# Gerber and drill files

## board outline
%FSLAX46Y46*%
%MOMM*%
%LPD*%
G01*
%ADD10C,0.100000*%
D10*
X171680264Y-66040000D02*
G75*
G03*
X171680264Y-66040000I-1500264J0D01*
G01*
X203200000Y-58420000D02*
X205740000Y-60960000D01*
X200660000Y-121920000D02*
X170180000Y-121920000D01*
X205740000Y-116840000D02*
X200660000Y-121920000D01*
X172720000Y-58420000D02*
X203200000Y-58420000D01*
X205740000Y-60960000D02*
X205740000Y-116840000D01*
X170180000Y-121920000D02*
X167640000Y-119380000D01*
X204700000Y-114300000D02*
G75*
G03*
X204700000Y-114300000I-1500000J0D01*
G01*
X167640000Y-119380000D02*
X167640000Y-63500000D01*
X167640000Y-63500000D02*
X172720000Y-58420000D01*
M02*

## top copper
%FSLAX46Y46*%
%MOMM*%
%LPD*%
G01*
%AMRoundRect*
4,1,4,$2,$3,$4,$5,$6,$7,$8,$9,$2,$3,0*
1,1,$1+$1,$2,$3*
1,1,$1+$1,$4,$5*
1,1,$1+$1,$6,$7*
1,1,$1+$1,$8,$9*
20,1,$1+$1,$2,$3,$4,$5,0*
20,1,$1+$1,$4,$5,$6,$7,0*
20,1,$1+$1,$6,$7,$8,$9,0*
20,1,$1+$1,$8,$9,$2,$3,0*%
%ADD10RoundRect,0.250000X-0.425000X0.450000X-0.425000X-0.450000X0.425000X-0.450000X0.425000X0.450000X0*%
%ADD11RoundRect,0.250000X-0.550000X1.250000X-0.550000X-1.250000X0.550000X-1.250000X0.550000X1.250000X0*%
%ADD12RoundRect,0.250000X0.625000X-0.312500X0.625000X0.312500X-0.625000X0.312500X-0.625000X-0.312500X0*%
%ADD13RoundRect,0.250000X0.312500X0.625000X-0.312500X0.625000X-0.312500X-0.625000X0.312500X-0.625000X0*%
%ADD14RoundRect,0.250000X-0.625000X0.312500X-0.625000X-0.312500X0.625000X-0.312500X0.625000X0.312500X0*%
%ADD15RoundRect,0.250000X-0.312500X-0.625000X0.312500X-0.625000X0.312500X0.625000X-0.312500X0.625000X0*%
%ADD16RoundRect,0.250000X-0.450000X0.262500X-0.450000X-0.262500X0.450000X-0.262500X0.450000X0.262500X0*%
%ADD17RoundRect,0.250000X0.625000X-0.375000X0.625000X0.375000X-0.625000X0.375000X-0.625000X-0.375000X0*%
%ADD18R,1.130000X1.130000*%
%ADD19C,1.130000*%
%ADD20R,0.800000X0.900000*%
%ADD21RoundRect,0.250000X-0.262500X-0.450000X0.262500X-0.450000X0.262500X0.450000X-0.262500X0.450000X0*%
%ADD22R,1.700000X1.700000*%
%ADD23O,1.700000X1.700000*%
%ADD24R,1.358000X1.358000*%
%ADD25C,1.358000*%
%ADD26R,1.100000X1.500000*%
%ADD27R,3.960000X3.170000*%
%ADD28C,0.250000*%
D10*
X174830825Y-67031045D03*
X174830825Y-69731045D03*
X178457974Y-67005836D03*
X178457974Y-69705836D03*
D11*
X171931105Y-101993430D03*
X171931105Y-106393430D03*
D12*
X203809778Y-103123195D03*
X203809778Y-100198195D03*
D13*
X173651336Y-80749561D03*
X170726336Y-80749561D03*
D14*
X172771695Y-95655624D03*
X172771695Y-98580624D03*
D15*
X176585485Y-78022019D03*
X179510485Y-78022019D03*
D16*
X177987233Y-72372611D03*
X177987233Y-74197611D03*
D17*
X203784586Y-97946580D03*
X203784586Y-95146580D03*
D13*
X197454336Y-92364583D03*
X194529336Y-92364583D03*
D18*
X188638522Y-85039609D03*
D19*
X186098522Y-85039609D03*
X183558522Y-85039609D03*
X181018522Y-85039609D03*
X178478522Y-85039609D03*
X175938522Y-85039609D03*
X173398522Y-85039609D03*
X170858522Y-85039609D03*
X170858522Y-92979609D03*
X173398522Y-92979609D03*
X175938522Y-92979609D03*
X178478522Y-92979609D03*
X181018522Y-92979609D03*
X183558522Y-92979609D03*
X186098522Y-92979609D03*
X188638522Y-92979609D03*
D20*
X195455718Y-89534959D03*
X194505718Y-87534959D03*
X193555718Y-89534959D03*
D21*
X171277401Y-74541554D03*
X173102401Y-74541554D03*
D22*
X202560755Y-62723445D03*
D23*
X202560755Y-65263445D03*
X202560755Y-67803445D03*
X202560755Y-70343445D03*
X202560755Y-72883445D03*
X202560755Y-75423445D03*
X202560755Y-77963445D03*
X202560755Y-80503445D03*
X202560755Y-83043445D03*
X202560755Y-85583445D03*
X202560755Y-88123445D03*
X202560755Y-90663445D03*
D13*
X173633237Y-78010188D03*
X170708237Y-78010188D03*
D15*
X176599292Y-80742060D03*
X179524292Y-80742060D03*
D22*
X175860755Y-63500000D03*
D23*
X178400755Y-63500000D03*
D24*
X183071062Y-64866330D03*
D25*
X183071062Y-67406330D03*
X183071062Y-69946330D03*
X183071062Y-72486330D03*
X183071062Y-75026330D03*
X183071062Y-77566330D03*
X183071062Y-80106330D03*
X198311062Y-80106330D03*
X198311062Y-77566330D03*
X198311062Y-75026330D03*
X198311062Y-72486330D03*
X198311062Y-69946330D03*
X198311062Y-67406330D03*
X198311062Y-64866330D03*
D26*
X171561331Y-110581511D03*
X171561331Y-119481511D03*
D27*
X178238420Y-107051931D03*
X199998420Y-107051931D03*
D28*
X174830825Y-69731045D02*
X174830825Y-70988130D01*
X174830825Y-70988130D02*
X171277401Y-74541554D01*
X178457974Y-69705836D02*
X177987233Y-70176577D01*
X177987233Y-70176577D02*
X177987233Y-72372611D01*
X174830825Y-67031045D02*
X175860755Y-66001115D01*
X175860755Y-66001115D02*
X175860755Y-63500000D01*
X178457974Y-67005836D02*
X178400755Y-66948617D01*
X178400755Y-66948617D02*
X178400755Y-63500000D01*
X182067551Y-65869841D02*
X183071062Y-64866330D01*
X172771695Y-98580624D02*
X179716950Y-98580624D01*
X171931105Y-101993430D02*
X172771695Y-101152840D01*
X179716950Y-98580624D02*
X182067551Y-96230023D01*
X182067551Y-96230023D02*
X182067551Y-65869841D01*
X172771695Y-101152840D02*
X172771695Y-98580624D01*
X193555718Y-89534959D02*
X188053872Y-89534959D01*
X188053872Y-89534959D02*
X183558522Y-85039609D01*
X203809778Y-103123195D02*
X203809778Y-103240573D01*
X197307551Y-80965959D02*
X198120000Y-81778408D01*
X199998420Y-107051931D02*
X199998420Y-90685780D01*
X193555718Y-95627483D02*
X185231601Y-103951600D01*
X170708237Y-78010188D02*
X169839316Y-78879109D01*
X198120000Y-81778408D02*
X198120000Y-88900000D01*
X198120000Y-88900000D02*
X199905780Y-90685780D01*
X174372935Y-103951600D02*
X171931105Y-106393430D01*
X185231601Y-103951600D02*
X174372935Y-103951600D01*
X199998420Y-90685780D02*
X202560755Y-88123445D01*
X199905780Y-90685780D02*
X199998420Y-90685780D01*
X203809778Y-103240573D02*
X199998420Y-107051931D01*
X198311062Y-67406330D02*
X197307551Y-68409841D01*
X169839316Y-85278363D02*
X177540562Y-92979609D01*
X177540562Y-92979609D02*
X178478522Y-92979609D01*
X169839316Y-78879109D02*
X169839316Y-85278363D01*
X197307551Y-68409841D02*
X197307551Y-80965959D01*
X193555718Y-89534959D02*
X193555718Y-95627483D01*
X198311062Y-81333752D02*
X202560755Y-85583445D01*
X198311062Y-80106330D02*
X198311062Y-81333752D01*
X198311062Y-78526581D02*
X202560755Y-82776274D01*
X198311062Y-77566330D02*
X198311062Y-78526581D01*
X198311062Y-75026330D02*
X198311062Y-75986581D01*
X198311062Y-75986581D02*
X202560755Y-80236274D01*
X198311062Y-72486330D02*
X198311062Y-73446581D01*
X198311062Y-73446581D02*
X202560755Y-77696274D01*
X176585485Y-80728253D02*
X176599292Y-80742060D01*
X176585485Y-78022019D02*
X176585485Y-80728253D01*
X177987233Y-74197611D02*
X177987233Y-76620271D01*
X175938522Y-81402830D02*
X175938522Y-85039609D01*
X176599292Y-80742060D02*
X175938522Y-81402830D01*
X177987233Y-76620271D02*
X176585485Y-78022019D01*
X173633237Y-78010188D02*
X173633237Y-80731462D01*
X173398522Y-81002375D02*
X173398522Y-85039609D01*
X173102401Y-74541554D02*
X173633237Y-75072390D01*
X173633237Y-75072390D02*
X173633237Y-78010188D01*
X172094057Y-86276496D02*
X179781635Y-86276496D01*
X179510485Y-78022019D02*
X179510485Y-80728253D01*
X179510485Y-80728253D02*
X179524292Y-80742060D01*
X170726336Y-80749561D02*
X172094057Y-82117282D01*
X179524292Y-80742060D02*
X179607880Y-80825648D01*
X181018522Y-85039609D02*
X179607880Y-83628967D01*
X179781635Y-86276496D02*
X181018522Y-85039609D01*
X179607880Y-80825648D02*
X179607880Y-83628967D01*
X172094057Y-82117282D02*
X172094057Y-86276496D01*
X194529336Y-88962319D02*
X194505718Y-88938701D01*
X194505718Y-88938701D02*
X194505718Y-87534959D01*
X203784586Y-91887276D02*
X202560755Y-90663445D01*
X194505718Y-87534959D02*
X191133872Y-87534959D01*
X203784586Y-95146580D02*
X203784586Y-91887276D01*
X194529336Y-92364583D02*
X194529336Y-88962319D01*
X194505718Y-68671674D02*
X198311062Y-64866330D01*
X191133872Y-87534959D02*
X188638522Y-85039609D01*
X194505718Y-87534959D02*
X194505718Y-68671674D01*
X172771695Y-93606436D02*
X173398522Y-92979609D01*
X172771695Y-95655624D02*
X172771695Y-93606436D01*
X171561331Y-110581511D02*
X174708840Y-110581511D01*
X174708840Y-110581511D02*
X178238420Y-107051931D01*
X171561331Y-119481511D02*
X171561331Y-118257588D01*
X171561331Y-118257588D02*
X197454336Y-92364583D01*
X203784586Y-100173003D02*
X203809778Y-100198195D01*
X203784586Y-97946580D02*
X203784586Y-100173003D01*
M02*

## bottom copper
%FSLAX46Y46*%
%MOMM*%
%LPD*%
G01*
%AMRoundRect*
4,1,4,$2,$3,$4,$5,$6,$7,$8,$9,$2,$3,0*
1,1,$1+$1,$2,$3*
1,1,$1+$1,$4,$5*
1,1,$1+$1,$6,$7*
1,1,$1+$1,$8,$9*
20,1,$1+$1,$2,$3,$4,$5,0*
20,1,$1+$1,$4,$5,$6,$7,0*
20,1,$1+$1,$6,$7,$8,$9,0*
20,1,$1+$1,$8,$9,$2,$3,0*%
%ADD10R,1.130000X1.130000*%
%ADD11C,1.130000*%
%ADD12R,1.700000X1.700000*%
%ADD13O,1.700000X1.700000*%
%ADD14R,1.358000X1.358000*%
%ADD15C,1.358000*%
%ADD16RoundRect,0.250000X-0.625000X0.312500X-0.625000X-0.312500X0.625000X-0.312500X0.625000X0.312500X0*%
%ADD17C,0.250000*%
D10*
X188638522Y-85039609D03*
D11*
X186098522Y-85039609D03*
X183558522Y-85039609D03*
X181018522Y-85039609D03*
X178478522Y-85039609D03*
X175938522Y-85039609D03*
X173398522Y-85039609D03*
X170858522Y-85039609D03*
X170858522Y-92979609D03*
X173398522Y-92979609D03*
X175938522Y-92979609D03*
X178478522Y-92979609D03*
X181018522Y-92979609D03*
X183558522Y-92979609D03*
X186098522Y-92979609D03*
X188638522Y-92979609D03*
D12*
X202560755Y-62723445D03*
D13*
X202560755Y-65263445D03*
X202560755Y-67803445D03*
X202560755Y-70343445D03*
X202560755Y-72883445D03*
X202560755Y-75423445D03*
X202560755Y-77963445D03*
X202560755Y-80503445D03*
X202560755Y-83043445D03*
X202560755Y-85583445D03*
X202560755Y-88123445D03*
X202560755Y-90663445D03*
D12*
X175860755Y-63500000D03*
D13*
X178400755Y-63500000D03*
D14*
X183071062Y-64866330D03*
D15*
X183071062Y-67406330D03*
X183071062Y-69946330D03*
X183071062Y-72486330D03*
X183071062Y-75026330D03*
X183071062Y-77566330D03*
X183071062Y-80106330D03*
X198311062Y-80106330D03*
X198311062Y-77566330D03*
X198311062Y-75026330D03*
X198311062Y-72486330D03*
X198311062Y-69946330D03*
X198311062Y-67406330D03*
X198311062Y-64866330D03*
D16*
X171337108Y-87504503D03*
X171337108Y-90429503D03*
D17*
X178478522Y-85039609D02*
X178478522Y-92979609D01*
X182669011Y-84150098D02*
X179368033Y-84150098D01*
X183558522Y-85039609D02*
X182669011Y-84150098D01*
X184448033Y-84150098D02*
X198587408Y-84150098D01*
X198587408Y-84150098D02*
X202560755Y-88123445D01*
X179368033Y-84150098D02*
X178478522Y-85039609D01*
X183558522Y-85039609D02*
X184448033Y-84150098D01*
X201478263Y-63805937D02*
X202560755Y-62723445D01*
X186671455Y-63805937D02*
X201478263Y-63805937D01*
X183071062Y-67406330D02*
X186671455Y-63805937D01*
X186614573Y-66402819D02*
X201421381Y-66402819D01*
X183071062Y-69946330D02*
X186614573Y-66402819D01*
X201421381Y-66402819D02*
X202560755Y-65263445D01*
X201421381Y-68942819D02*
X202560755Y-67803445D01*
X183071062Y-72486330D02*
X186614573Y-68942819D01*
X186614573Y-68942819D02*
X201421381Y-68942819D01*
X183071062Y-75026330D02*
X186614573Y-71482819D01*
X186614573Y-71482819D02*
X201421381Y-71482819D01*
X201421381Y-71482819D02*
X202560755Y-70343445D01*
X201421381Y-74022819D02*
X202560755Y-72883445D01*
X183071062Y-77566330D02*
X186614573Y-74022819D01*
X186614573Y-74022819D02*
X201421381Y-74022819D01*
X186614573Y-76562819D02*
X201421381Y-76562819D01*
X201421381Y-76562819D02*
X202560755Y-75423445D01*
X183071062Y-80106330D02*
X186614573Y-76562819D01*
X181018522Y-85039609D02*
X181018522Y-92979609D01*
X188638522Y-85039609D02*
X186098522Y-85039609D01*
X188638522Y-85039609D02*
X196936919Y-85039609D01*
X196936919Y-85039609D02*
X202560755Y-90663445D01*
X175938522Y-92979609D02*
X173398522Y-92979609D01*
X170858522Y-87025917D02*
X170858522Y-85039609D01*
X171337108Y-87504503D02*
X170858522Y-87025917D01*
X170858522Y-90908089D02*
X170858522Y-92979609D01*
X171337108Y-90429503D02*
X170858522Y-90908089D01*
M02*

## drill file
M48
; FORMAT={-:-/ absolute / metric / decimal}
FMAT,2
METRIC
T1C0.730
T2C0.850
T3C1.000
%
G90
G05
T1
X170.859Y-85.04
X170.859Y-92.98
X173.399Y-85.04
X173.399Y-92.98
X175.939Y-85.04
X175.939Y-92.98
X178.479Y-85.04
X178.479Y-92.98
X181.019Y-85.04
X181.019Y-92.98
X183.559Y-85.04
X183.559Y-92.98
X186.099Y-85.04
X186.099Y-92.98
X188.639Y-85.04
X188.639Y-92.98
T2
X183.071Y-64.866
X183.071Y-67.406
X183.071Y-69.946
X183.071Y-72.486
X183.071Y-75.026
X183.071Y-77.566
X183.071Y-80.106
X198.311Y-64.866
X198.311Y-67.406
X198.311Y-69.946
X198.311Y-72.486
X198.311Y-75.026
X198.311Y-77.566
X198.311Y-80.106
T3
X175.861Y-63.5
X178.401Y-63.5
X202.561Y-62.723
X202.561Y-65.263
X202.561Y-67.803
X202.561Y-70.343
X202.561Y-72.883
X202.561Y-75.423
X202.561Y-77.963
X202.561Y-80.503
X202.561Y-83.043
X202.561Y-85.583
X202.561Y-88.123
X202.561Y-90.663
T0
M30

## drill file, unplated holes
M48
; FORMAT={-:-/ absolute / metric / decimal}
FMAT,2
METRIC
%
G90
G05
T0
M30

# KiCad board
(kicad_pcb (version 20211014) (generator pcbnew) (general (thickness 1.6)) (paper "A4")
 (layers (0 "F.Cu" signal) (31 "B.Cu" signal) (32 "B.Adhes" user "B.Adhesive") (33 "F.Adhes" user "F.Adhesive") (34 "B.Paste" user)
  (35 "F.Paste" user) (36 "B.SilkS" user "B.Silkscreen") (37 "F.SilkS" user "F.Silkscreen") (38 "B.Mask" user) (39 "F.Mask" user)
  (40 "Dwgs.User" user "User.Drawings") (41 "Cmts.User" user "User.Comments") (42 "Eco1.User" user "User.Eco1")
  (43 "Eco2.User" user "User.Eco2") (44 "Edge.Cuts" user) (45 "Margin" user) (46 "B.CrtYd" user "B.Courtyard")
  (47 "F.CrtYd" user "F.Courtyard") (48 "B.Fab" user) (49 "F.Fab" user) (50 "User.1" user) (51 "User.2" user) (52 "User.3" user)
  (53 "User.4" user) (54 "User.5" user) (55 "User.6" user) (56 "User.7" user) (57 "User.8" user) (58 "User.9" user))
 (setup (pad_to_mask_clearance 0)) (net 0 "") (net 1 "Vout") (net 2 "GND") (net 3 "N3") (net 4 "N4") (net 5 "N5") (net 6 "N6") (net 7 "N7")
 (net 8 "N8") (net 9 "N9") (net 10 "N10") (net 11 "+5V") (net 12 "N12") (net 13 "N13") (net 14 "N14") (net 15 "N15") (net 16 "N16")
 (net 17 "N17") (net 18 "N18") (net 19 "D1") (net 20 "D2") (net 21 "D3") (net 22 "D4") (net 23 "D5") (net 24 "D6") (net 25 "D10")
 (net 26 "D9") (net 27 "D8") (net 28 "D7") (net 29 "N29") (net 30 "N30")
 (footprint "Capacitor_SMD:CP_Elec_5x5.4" (layer "F.Cu") (at 171.931105 104.19343 -90)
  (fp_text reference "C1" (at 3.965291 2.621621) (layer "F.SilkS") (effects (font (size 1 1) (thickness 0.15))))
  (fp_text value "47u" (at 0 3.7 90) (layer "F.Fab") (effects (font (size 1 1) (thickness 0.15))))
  (pad "1" smd roundrect (at -2.2 0 270) (size 3 1.6) (layers "F.Cu" "F.Paste" "F.Mask") (roundrect_rratio 0.15625) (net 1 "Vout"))
  (pad "2" smd roundrect (at 2.2 0 270) (size 3 1.6) (layers "F.Cu" "F.Paste" "F.Mask") (roundrect_rratio 0.15625) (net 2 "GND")))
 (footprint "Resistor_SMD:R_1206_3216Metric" (layer "F.Cu") (at 203.809778 101.660695 90)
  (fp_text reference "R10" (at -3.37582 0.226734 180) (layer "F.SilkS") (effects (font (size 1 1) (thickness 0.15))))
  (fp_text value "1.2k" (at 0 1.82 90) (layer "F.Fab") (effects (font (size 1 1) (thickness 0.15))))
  (pad "1" smd roundrect (at -1.4625 0 90) (size 1.125 1.75) (layers "F.Cu" "F.Paste" "F.Mask") (roundrect_rratio 0.2222222222)
   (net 2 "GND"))
  (pad "2" smd roundrect (at 1.4625 0 90) (size 1.125 1.75) (layers "F.Cu" "F.Paste" "F.Mask") (roundrect_rratio 0.2222222222) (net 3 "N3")))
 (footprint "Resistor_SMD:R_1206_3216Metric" (layer "F.Cu") (at 172.188836 80.749561 180)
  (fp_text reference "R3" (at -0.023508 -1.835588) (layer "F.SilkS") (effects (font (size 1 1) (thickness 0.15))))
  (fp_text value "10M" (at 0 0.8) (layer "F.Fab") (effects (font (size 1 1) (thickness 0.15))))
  (pad "1" smd roundrect (at -1.4625 0 180) (size 1.125 1.75) (layers "F.Cu" "F.Paste" "F.Mask") (roundrect_rratio 0.2222222222)
   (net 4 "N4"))
  (pad "2" smd roundrect (at 1.4625 0 180) (size 1.125 1.75) (layers "F.Cu" "F.Paste" "F.Mask") (roundrect_rratio 0.2222222222) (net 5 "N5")))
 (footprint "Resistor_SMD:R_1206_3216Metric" (layer "F.Cu") (at 172.771695 97.118124 -90)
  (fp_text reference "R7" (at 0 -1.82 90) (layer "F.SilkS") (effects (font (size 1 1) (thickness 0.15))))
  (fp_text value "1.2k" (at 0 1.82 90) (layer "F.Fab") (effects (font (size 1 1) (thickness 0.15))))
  (pad "1" smd roundrect (at -1.4625 0 270) (size 1.125 1.75) (layers "F.Cu" "F.Paste" "F.Mask") (roundrect_rratio 0.2222222222)
   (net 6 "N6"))
  (pad "2" smd roundrect (at 1.4625 0 270) (size 1.125 1.75) (layers "F.Cu" "F.Paste" "F.Mask") (roundrect_rratio 0.2222222222)
   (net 1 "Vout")))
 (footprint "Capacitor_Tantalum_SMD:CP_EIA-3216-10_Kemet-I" (layer "F.Cu") (at 174.830825 68.381045 -90)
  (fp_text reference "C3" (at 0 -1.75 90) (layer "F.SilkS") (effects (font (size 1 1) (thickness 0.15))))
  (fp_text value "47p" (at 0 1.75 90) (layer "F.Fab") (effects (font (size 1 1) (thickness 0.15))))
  (pad "1" smd roundrect (at -1.35 0 270) (size 1.4 1.35) (layers "F.Cu" "F.Paste" "F.Mask") (roundrect_rratio 0.1851851852) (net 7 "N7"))
  (pad "2" smd roundrect (at 1.35 0 270) (size 1.4 1.35) (layers "F.Cu" "F.Paste" "F.Mask") (roundrect_rratio 0.1851851852) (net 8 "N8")))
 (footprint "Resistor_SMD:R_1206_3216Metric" (layer "F.Cu") (at 178.047985 78.022019)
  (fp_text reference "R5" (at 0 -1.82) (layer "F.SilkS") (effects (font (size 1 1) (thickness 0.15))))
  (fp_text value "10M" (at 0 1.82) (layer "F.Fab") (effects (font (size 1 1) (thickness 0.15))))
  (pad "1" smd roundrect (at -1.4625 0) (size 1.125 1.75) (layers "F.Cu" "F.Paste" "F.Mask") (roundrect_rratio 0.2222222222) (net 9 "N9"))
  (pad "2" smd roundrect (at 1.4625 0) (size 1.125 1.75) (layers "F.Cu" "F.Paste" "F.Mask") (roundrect_rratio 0.2222222222) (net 5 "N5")))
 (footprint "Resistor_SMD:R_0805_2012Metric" (layer "F.Cu") (at 177.987233 73.285111 -90)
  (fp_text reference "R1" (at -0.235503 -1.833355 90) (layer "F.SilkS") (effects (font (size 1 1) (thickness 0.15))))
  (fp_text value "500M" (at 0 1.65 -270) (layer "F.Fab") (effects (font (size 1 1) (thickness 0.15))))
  (pad "1" smd roundrect (at -0.9125 0 270) (size 1.025 1.4) (layers "F.Cu" "F.Paste" "F.Mask") (roundrect_rratio 0.243902439)
   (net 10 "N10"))
  (pad "2" smd roundrect (at 0.9125 0 270) (size 1.025 1.4) (layers "F.Cu" "F.Paste" "F.Mask") (roundrect_rratio 0.243902439) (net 9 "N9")))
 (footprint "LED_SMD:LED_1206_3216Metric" (layer "F.Cu") (at 203.784586 96.54658 90)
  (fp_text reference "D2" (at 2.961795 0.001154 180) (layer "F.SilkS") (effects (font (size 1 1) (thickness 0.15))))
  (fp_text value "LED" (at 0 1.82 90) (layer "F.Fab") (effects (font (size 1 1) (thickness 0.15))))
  (pad "1" smd roundrect (at -1.4 0 90) (size 1.25 1.75) (layers "F.Cu" "F.Paste" "F.Mask") (roundrect_rratio 0.2) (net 3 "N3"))
  (pad "2" smd roundrect (at 1.4 0 90) (size 1.25 1.75) (layers "F.Cu" "F.Paste" "F.Mask") (roundrect_rratio 0.2) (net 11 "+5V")))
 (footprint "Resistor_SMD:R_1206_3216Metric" (layer "F.Cu") (at 195.991836 92.364583 180)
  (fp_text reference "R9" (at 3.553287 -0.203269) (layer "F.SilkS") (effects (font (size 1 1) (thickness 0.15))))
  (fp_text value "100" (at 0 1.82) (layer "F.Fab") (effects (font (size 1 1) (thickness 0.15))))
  (pad "1" smd roundrect (at -1.4625 0 180) (size 1.125 1.75) (layers "F.Cu" "F.Paste" "F.Mask") (roundrect_rratio 0.2222222222)
   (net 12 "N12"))
  (pad "2" smd roundrect (at 1.4625 0 180) (size 1.125 1.75) (layers "F.Cu" "F.Paste" "F.Mask") (roundrect_rratio 0.2222222222)
   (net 11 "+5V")))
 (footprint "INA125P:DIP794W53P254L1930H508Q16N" (layer "F.Cu") (at 179.748522 89.009609 -90)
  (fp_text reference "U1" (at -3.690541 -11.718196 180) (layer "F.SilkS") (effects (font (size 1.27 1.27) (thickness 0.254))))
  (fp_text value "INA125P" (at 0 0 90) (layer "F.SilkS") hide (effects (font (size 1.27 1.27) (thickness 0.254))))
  (pad "1" thru_hole rect locked (at -3.97 -8.89 270) (size 1.13 1.13) (drill 0.73) (layers *.Cu *.Mask) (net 11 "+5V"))
  (pad "2" thru_hole circle locked (at -3.97 -6.35 270) (size 1.13 1.13) (drill 0.73) (layers *.Cu *.Mask) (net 11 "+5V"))
  (pad "3" thru_hole circle locked (at -3.97 -3.81 270) (size 1.13 1.13) (drill 0.73) (layers *.Cu *.Mask) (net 2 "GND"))
  (pad "4" thru_hole circle locked (at -3.97 -1.27 270) (size 1.13 1.13) (drill 0.73) (layers *.Cu *.Mask) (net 5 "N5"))
  (pad "5" thru_hole circle locked (at -3.97 1.27 270) (size 1.13 1.13) (drill 0.73) (layers *.Cu *.Mask) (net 2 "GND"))
  (pad "6" thru_hole circle locked (at -3.97 3.81 270) (size 1.13 1.13) (drill 0.73) (layers *.Cu *.Mask) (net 9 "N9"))
  (pad "7" thru_hole circle locked (at -3.97 6.35 270) (size 1.13 1.13) (drill 0.73) (layers *.Cu *.Mask) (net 4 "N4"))
  (pad "8" thru_hole circle locked (at -3.97 8.89 270) (size 1.13 1.13) (drill 0.73) (layers *.Cu *.Mask) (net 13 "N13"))
  (pad "9" thru_hole circle locked (at 3.97 8.89 270) (size 1.13 1.13) (drill 0.73) (layers *.Cu *.Mask) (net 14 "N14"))
  (pad "10" thru_hole circle locked (at 3.97 6.35 270) (size 1.13 1.13) (drill 0.73) (layers *.Cu *.Mask) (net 6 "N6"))
  (pad "11" thru_hole circle locked (at 3.97 3.81 270) (size 1.13 1.13) (drill 0.73) (layers *.Cu *.Mask) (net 6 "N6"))
  (pad "12" thru_hole circle locked (at 3.97 1.27 270) (size 1.13 1.13) (drill 0.73) (layers *.Cu *.Mask) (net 2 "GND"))
  (pad "13" thru_hole circle locked (at 3.97 -1.27 270) (size 1.13 1.13) (drill 0.73) (layers *.Cu *.Mask) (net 5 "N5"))
  (pad "14" thru_hole circle locked (at 3.97 -3.81 270) (size 1.13 1.13) (drill 0.73) (layers *.Cu *.Mask) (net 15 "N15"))
  (pad "15" thru_hole circle locked (at 3.97 -6.35 270) (size 1.13 1.13) (drill 0.73) (layers *.Cu *.Mask) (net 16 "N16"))
  (pad "16" thru_hole circle locked (at 3.97 -8.89 270) (size 1.13 1.13) (drill 0.73) (layers *.Cu *.Mask) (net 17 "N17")))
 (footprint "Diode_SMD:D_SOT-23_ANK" (layer "F.Cu") (at 194.505718 88.534959 90)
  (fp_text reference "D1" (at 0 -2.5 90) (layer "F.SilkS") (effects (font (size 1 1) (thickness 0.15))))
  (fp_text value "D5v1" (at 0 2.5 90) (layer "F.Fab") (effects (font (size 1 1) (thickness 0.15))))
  (pad "" smd rect (at -1 0.95 90) (size 0.9 0.8) (layers "F.Cu" "F.Paste" "F.Mask"))
  (pad "1" smd rect (at 1 0 90) (size 0.9 0.8) (layers "F.Cu" "F.Paste" "F.Mask") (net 11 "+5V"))
  (pad "2" smd rect (at -1 -0.95 90) (size 0.9 0.8) (layers "F.Cu" "F.Paste" "F.Mask") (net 2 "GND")))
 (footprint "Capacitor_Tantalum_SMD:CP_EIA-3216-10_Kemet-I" (layer "F.Cu") (at 178.457974 68.355836 -90)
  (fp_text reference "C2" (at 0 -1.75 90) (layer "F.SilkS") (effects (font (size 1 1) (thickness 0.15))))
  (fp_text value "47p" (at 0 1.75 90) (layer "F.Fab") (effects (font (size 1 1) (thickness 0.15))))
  (pad "1" smd roundrect (at -1.35 0 270) (size 1.4 1.35) (layers "F.Cu" "F.Paste" "F.Mask") (roundrect_rratio 0.1851851852) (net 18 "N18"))
  (pad "2" smd roundrect (at 1.35 0 270) (size 1.4 1.35) (layers "F.Cu" "F.Paste" "F.Mask") (roundrect_rratio 0.1851851852) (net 10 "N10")))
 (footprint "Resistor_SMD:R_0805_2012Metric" (layer "F.Cu") (at 172.189901 74.541554)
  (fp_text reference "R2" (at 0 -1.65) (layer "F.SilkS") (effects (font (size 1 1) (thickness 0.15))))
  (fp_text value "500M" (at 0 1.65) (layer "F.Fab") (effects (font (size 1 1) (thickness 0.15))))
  (pad "1" smd roundrect (at -0.9125 0) (size 1.025 1.4) (layers "F.Cu" "F.Paste" "F.Mask") (roundrect_rratio 0.243902439) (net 8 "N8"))
  (pad "2" smd roundrect (at 0.9125 0) (size 1.025 1.4) (layers "F.Cu" "F.Paste" "F.Mask") (roundrect_rratio 0.243902439) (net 4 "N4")))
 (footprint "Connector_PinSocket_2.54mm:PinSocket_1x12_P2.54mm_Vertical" (layer "F.Cu") (at 202.560755 62.723445)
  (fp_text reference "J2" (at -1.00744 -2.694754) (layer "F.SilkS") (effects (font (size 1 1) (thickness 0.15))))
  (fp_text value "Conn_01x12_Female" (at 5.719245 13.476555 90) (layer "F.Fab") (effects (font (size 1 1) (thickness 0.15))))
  (pad "1" thru_hole rect (at 0 0) (size 1.7 1.7) (drill 1) (layers *.Cu *.Mask) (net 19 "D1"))
  (pad "2" thru_hole oval (at 0 2.54) (size 1.7 1.7) (drill 1) (layers *.Cu *.Mask) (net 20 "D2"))
  (pad "3" thru_hole oval (at 0 5.08) (size 1.7 1.7) (drill 1) (layers *.Cu *.Mask) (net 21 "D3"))
  (pad "4" thru_hole oval (at 0 7.62) (size 1.7 1.7) (drill 1) (layers *.Cu *.Mask) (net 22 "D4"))
  (pad "5" thru_hole oval (at 0 10.16) (size 1.7 1.7) (drill 1) (layers *.Cu *.Mask) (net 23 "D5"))
  (pad "6" thru_hole oval (at 0 12.7) (size 1.7 1.7) (drill 1) (layers *.Cu *.Mask) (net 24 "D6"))
  (pad "7" thru_hole oval (at 0 15.24) (size 1.7 1.7) (drill 1) (layers *.Cu *.Mask) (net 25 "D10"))
  (pad "8" thru_hole oval (at 0 17.78) (size 1.7 1.7) (drill 1) (layers *.Cu *.Mask) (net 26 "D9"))
  (pad "9" thru_hole oval (at 0 20.32) (size 1.7 1.7) (drill 1) (layers *.Cu *.Mask) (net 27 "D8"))
  (pad "10" thru_hole oval (at 0 22.86) (size 1.7 1.7) (drill 1) (layers *.Cu *.Mask) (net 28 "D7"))
  (pad "11" thru_hole oval (at 0 25.4) (size 1.7 1.7) (drill 1) (layers *.Cu *.Mask) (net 2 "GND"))
  (pad "12" thru_hole oval (at 0 27.94) (size 1.7 1.7) (drill 1) (layers *.Cu *.Mask) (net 11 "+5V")))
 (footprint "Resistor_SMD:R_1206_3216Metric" (layer "F.Cu") (at 172.170737 78.010188 180)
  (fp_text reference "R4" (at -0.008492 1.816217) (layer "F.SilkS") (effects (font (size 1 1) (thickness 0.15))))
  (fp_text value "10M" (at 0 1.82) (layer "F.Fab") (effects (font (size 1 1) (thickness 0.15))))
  (pad "1" smd roundrect (at -1.4625 0 180) (size 1.125 1.75) (layers "F.Cu" "F.Paste" "F.Mask") (roundrect_rratio 0.2222222222)
   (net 4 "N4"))
  (pad "2" smd roundrect (at 1.4625 0 180) (size 1.125 1.75) (layers "F.Cu" "F.Paste" "F.Mask") (roundrect_rratio 0.2222222222)
   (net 2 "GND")))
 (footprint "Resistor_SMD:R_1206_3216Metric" (layer "F.Cu") (at 178.061792 80.74206)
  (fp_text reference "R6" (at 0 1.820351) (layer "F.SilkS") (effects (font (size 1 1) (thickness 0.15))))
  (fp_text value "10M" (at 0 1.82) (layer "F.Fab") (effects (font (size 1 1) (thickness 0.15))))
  (pad "1" smd roundrect (at -1.4625 0) (size 1.125 1.75) (layers "F.Cu" "F.Paste" "F.Mask") (roundrect_rratio 0.2222222222) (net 9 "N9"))
  (pad "2" smd roundrect (at 1.4625 0) (size 1.125 1.75) (layers "F.Cu" "F.Paste" "F.Mask") (roundrect_rratio 0.2222222222) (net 5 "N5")))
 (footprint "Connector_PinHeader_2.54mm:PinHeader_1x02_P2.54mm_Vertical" (layer "F.Cu") (at 175.860755 63.5 90)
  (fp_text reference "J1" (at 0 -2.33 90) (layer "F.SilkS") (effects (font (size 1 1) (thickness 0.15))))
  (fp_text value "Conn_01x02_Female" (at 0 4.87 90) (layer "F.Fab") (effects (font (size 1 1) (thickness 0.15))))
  (pad "1" thru_hole rect (at 0 0 90) (size 1.7 1.7) (drill 1) (layers *.Cu *.Mask) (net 7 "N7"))
  (pad "2" thru_hole oval (at 0 2.54 90) (size 1.7 1.7) (drill 1) (layers *.Cu *.Mask) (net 18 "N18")))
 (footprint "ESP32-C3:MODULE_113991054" (layer "F.Cu") (at 190.691062 72.42283)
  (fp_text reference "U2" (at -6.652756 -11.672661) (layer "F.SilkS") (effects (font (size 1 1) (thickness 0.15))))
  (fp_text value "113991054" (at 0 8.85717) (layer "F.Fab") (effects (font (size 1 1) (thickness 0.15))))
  (pad "1" thru_hole rect locked (at -7.62 -7.5565) (size 1.358 1.358) (drill 0.85) (layers *.Cu *.Mask) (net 1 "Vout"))
  (pad "2" thru_hole circle locked (at -7.62 -5.0165) (size 1.358 1.358) (drill 0.85) (layers *.Cu *.Mask) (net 19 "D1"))
  (pad "3" thru_hole circle locked (at -7.62 -2.4765) (size 1.358 1.358) (drill 0.85) (layers *.Cu *.Mask) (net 20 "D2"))
  (pad "4" thru_hole circle locked (at -7.62 0.0635) (size 1.358 1.358) (drill 0.85) (layers *.Cu *.Mask) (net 21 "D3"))
  (pad "5" thru_hole circle locked (at -7.62 2.6035) (size 1.358 1.358) (drill 0.85) (layers *.Cu *.Mask) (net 22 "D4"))
  (pad "6" thru_hole circle locked (at -7.62 5.1435) (size 1.358 1.358) (drill 0.85) (layers *.Cu *.Mask) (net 23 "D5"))
  (pad "7" thru_hole circle locked (at -7.62 7.6835) (size 1.358 1.358) (drill 0.85) (layers *.Cu *.Mask) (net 24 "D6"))
  (pad "8" thru_hole circle locked (at 7.62 7.6835) (size 1.358 1.358) (drill 0.85) (layers *.Cu *.Mask) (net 28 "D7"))
  (pad "9" thru_hole circle locked (at 7.62 5.1435) (size 1.358 1.358) (drill 0.85) (layers *.Cu *.Mask) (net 27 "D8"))
  (pad "10" thru_hole circle locked (at 7.62 2.6035) (size 1.358 1.358) (drill 0.85) (layers *.Cu *.Mask) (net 26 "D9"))
  (pad "11" thru_hole circle locked (at 7.62 0.0635) (size 1.358 1.358) (drill 0.85) (layers *.Cu *.Mask) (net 25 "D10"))
  (pad "12" thru_hole circle locked (at 7.62 -2.4765) (size 1.358 1.358) (drill 0.85) (layers *.Cu *.Mask) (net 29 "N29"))
  (pad "13" thru_hole circle locked (at 7.62 -5.0165) (size 1.358 1.358) (drill 0.85) (layers *.Cu *.Mask) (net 2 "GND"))
  (pad "14" thru_hole circle locked (at 7.62 -7.5565) (size 1.358 1.358) (drill 0.85) (layers *.Cu *.Mask) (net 11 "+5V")))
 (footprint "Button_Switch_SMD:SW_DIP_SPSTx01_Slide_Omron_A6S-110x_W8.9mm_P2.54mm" (layer "F.Cu") (at 171.561331 115.031511 -90)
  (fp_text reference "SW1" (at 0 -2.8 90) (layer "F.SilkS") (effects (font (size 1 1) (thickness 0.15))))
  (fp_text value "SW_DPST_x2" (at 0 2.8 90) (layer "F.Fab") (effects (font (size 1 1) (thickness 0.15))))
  (pad "1" smd rect (at -4.45 0 270) (size 1.5 1.1) (layers "F.Cu" "F.Paste" "F.Mask") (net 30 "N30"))
  (pad "2" smd rect (at 4.45 0 270) (size 1.5 1.1) (layers "F.Cu" "F.Paste" "F.Mask") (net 12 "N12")))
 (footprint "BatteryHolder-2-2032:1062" (layer "F.Cu") (at 189.11842 107.051931 -90)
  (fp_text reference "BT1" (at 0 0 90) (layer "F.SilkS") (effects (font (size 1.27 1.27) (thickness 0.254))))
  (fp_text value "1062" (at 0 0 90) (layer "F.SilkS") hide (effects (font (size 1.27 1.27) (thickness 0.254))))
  (pad "1" smd rect locked (at 0 10.88 270) (size 3.17 3.96) (layers "F.Cu" "F.Paste" "F.Mask") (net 30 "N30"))
  (pad "2" smd rect locked (at 0 -10.88 270) (size 3.17 3.96) (layers "F.Cu" "F.Paste" "F.Mask") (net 2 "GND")))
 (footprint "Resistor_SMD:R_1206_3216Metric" (layer "B.Cu") (at 171.337108 88.967003 -90)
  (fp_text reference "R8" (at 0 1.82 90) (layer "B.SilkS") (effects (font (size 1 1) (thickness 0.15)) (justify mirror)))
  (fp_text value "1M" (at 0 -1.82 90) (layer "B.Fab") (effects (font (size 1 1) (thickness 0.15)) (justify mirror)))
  (pad "1" smd roundrect (at -1.4625 0 270) (size 1.125 1.75) (layers "B.Cu" "B.Paste" "B.Mask") (roundrect_rratio 0.2222222222)
   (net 13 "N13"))
  (pad "2" smd roundrect (at 1.4625 0 270) (size 1.125 1.75) (layers "B.Cu" "B.Paste" "B.Mask") (roundrect_rratio 0.2222222222)
   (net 14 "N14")))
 (gr_circle (center 170.18 66.04) (end 168.681434 66.11136) (layer "Edge.Cuts") (width 0.1) (fill none))
 (gr_line (start 203.2 58.42) (end 205.74 60.96) (layer "Edge.Cuts") (width 0.1))
 (gr_line (start 200.66 121.92) (end 170.18 121.92) (layer "Edge.Cuts") (width 0.1))
 (gr_line (start 205.74 116.84) (end 200.66 121.92) (layer "Edge.Cuts") (width 0.1))
 (gr_line (start 172.72 58.42) (end 203.2 58.42) (layer "Edge.Cuts") (width 0.1))
 (gr_line (start 205.74 60.96) (end 205.74 116.84) (layer "Edge.Cuts") (width 0.1))
 (gr_line (start 170.18 121.92) (end 167.64 119.38) (layer "Edge.Cuts") (width 0.1))
 (gr_circle (center 203.2 114.3) (end 204.7 114.3) (layer "Edge.Cuts") (width 0.1) (fill none))
 (gr_line (start 167.64 119.38) (end 167.64 63.5) (layer "Edge.Cuts") (width 0.1))
 (gr_line (start 167.64 63.5) (end 172.72 58.42) (layer "Edge.Cuts") (width 0.1))
 (segment (start 182.067551 65.869841) (end 183.071062 64.86633) (width 0.25) (layer "F.Cu") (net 1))
 (segment (start 172.771695 98.580624) (end 179.71695 98.580624) (width 0.25) (layer "F.Cu") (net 1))
 (segment (start 171.931105 101.99343) (end 172.771695 101.15284) (width 0.25) (layer "F.Cu") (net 1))
 (segment (start 179.71695 98.580624) (end 182.067551 96.230023) (width 0.25) (layer "F.Cu") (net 1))
 (segment (start 182.067551 96.230023) (end 182.067551 65.869841) (width 0.25) (layer "F.Cu") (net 1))
 (segment (start 172.771695 101.15284) (end 172.771695 98.580624) (width 0.25) (layer "F.Cu") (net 1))
 (segment (start 193.555718 89.534959) (end 188.053872 89.534959) (width 0.25) (layer "F.Cu") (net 2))
 (segment (start 188.053872 89.534959) (end 183.558522 85.039609) (width 0.25) (layer "F.Cu") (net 2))
 (segment (start 203.809778 103.123195) (end 203.809778 103.240573) (width 0.25) (layer "F.Cu") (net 2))
 (segment (start 197.307551 80.965959) (end 198.12 81.778408) (width 0.25) (layer "F.Cu") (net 2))
 (segment (start 199.99842 107.051931) (end 199.99842 90.68578) (width 0.25) (layer "F.Cu") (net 2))
 (segment (start 193.555718 95.627483) (end 185.231601 103.9516) (width 0.25) (layer "F.Cu") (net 2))
 (segment (start 170.708237 78.010188) (end 169.839316 78.879109) (width 0.25) (layer "F.Cu") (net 2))
 (segment (start 198.12 81.778408) (end 198.12 88.9) (width 0.25) (layer "F.Cu") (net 2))
 (segment (start 198.12 88.9) (end 199.90578 90.68578) (width 0.25) (layer "F.Cu") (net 2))
 (segment (start 174.372935 103.9516) (end 171.931105 106.39343) (width 0.25) (layer "F.Cu") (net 2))
 (segment (start 185.231601 103.9516) (end 174.372935 103.9516) (width 0.25) (layer "F.Cu") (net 2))
 (segment (start 199.99842 90.68578) (end 202.560755 88.123445) (width 0.25) (layer "F.Cu") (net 2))
 (segment (start 199.90578 90.68578) (end 199.99842 90.68578) (width 0.25) (layer "F.Cu") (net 2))
 (segment (start 203.809778 103.240573) (end 199.99842 107.051931) (width 0.25) (layer "F.Cu") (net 2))
 (segment (start 198.311062 67.40633) (end 197.307551 68.409841) (width 0.25) (layer "F.Cu") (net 2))
 (segment (start 169.839316 85.278363) (end 177.540562 92.979609) (width 0.25) (layer "F.Cu") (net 2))
 (segment (start 177.540562 92.979609) (end 178.478522 92.979609) (width 0.25) (layer "F.Cu") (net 2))
 (segment (start 169.839316 78.879109) (end 169.839316 85.278363) (width 0.25) (layer "F.Cu") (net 2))
 (segment (start 197.307551 68.409841) (end 197.307551 80.965959) (width 0.25) (layer "F.Cu") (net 2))
 (segment (start 193.555718 89.534959) (end 193.555718 95.627483) (width 0.25) (layer "F.Cu") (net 2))
 (segment (start 178.478522 85.039609) (end 178.478522 92.979609) (width 0.25) (layer "B.Cu") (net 2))
 (segment (start 182.669011 84.150098) (end 179.368033 84.150098) (width 0.25) (layer "B.Cu") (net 2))
 (segment (start 183.558522 85.039609) (end 182.669011 84.150098) (width 0.25) (layer "B.Cu") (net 2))
 (segment (start 184.448033 84.150098) (end 198.587408 84.150098) (width 0.25) (layer "B.Cu") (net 2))
 (segment (start 198.587408 84.150098) (end 202.560755 88.123445) (width 0.25) (layer "B.Cu") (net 2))
 (segment (start 179.368033 84.150098) (end 178.478522 85.039609) (width 0.25) (layer "B.Cu") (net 2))
 (segment (start 183.558522 85.039609) (end 184.448033 84.150098) (width 0.25) (layer "B.Cu") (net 2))
 (segment (start 201.478263 63.805937) (end 202.560755 62.723445) (width 0.25) (layer "B.Cu") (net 19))
 (segment (start 186.671455 63.805937) (end 201.478263 63.805937) (width 0.25) (layer "B.Cu") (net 19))
 (segment (start 183.071062 67.40633) (end 186.671455 63.805937) (width 0.25) (layer "B.Cu") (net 19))
 (segment (start 186.614573 66.402819) (end 201.421381 66.402819) (width 0.25) (layer "B.Cu") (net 20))
 (segment (start 183.071062 69.94633) (end 186.614573 66.402819) (width 0.25) (layer "B.Cu") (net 20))
 (segment (start 201.421381 66.402819) (end 202.560755 65.263445) (width 0.25) (layer "B.Cu") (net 20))
 (segment (start 201.421381 68.942819) (end 202.560755 67.803445) (width 0.25) (layer "B.Cu") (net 21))
 (segment (start 183.071062 72.48633) (end 186.614573 68.942819) (width 0.25) (layer "B.Cu") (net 21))
 (segment (start 186.614573 68.942819) (end 201.421381 68.942819) (width 0.25) (layer "B.Cu") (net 21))
 (segment (start 183.071062 75.02633) (end 186.614573 71.482819) (width 0.25) (layer "B.Cu") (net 22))
 (segment (start 186.614573 71.482819) (end 201.421381 71.482819) (width 0.25) (layer "B.Cu") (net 22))
 (segment (start 201.421381 71.482819) (end 202.560755 70.343445) (width 0.25) (layer "B.Cu") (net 22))
 (segment (start 201.421381 74.022819) (end 202.560755 72.883445) (width 0.25) (layer "B.Cu") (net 23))
 (segment (start 183.071062 77.56633) (end 186.614573 74.022819) (width 0.25) (layer "B.Cu") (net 23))
 (segment (start 186.614573 74.022819) (end 201.421381 74.022819) (width 0.25) (layer "B.Cu") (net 23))
 (segment (start 186.614573 76.562819) (end 201.421381 76.562819) (width 0.25) (layer "B.Cu") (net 24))
 (segment (start 201.421381 76.562819) (end 202.560755 75.423445) (width 0.25) (layer "B.Cu") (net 24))
 (segment (start 183.071062 80.10633) (end 186.614573 76.562819) (width 0.25) (layer "B.Cu") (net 24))
 (segment (start 198.311062 81.333752) (end 202.560755 85.583445) (width 0.25) (layer "F.Cu") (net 28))
 (segment (start 198.311062 80.10633) (end 198.311062 81.333752) (width 0.25) (layer "F.Cu") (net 28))
 (segment (start 198.311062 78.526581) (end 202.560755 82.776274) (width 0.25) (layer "F.Cu") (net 27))
 (segment (start 198.311062 77.56633) (end 198.311062 78.526581) (width 0.25) (layer "F.Cu") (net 27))
 (segment (start 198.311062 75.02633) (end 198.311062 75.986581) (width 0.25) (layer "F.Cu") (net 26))
 (segment (start 198.311062 75.986581) (end 202.560755 80.236274) (width 0.25) (layer "F.Cu") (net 26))
 (segment (start 198.311062 72.48633) (end 198.311062 73.446581) (width 0.25) (layer "F.Cu") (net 25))
 (segment (start 198.311062 73.446581) (end 202.560755 77.696274) (width 0.25) (layer "F.Cu") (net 25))
 (segment (start 176.585485 80.728253) (end 176.599292 80.74206) (width 0.25) (layer "F.Cu") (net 9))
 (segment (start 176.585485 78.022019) (end 176.585485 80.728253) (width 0.25) (layer "F.Cu") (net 9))
 (segment (start 177.987233 74.197611) (end 177.987233 76.620271) (width 0.25) (layer "F.Cu") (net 9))
 (segment (start 175.938522 81.40283) (end 175.938522 85.039609) (width 0.25) (layer "F.Cu") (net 9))
 (segment (start 176.599292 80.74206) (end 175.938522 81.40283) (width 0.25) (layer "F.Cu") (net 9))
 (segment (start 177.987233 76.620271) (end 176.585485 78.022019) (width 0.25) (layer "F.Cu") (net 9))
 (segment (start 173.633237 78.010188) (end 173.633237 80.731462) (width 0.25) (layer "F.Cu") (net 4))
 (segment (start 173.398522 81.002375) (end 173.398522 85.039609) (width 0.25) (layer "F.Cu") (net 4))
 (segment (start 173.102401 74.541554) (end 173.633237 75.07239) (width 0.25) (layer "F.Cu") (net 4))
 (segment (start 173.633237 75.07239) (end 173.633237 78.010188) (width 0.25) (layer "F.Cu") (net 4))
 (segment (start 172.094057 86.276496) (end 179.781635 86.276496) (width 0.25) (layer "F.Cu") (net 5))
 (segment (start 179.510485 78.022019) (end 179.510485 80.728253) (width 0.25) (layer "F.Cu") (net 5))
 (segment (start 179.510485 80.728253) (end 179.524292 80.74206) (width 0.25) (layer "F.Cu") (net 5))
 (segment (start 170.726336 80.749561) (end 172.094057 82.117282) (width 0.25) (layer "F.Cu") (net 5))
 (segment (start 179.524292 80.74206) (end 179.60788 80.825648) (width 0.25) (layer "F.Cu") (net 5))
 (segment (start 181.018522 85.039609) (end 179.60788 83.628967) (width 0.25) (layer "F.Cu") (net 5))
 (segment (start 179.781635 86.276496) (end 181.018522 85.039609) (width 0.25) (layer "F.Cu") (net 5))
 (segment (start 179.60788 80.825648) (end 179.60788 83.628967) (width 0.25) (layer "F.Cu") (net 5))
 (segment (start 172.094057 82.117282) (end 172.094057 86.276496) (width 0.25) (layer "F.Cu") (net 5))
 (segment (start 181.018522 85.039609) (end 181.018522 92.979609) (width 0.25) (layer "B.Cu") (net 5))
 (segment (start 194.529336 88.962319) (end 194.505718 88.938701) (width 0.25) (layer "F.Cu") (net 11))
 (segment (start 194.505718 88.938701) (end 194.505718 87.534959) (width 0.25) (layer "F.Cu") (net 11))
 (segment (start 203.784586 91.887276) (end 202.560755 90.663445) (width 0.25) (layer "F.Cu") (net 11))
 (segment (start 194.505718 87.534959) (end 191.133872 87.534959) (width 0.25) (layer "F.Cu") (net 11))
 (segment (start 203.784586 95.14658) (end 203.784586 91.887276) (width 0.25) (layer "F.Cu") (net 11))
 (segment (start 194.529336 92.364583) (end 194.529336 88.962319) (width 0.25) (layer "F.Cu") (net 11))
 (segment (start 194.505718 68.671674) (end 198.311062 64.86633) (width 0.25) (layer "F.Cu") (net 11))
 (segment (start 191.133872 87.534959) (end 188.638522 85.039609) (width 0.25) (layer "F.Cu") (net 11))
 (segment (start 194.505718 87.534959) (end 194.505718 68.671674) (width 0.25) (layer "F.Cu") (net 11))
 (segment (start 188.638522 85.039609) (end 186.098522 85.039609) (width 0.25) (layer "B.Cu") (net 11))
 (segment (start 188.638522 85.039609) (end 196.936919 85.039609) (width 0.25) (layer "B.Cu") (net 11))
 (segment (start 196.936919 85.039609) (end 202.560755 90.663445) (width 0.25) (layer "B.Cu") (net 11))
 (segment (start 172.771695 93.606436) (end 173.398522 92.979609) (width 0.25) (layer "F.Cu") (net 6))
 (segment (start 172.771695 95.655624) (end 172.771695 93.606436) (width 0.25) (layer "F.Cu") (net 6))
 (segment (start 175.938522 92.979609) (end 173.398522 92.979609) (width 0.25) (layer "B.Cu") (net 6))
 (segment (start 175.860755 66.001115) (end 175.860755 63.5) (width 0.25) (layer "F.Cu") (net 7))
 (segment (start 174.830825 67.031045) (end 175.860755 66.001115) (width 0.25) (layer "F.Cu") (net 7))
 (segment (start 178.400755 66.948617) (end 178.400755 63.5) (width 0.25) (layer "F.Cu") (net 18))
 (segment (start 178.457974 67.005836) (end 178.400755 66.948617) (width 0.25) (layer "F.Cu") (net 18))
 (segment (start 170.858522 87.025917) (end 170.858522 85.039609) (width 0.25) (layer "B.Cu") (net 13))
 (segment (start 171.337108 87.504503) (end 170.858522 87.025917) (width 0.25) (layer "B.Cu") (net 13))
 (segment (start 171.561331 110.581511) (end 174.70884 110.581511) (width 0.25) (layer "F.Cu") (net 30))
 (segment (start 174.70884 110.581511) (end 178.23842 107.051931) (width 0.25) (layer "F.Cu") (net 30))
 (segment (start 170.858522 90.908089) (end 170.858522 92.979609) (width 0.25) (layer "B.Cu") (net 14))
 (segment (start 171.337108 90.429503) (end 170.858522 90.908089) (width 0.25) (layer "B.Cu") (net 14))
 (segment (start 171.561331 119.481511) (end 171.561331 118.257588) (width 0.25) (layer "F.Cu") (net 12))
 (segment (start 171.561331 118.257588) (end 197.454336 92.364583) (width 0.25) (layer "F.Cu") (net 12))
 (segment (start 203.784586 100.173003) (end 203.809778 100.198195) (width 0.25) (layer "F.Cu") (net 3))
 (segment (start 203.784586 97.94658) (end 203.784586 100.173003) (width 0.25) (layer "F.Cu") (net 3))
 (segment (start 177.987233 70.176577) (end 177.987233 72.372611) (width 0.25) (layer "F.Cu") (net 10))
 (segment (start 178.457974 69.705836) (end 177.987233 70.176577) (width 0.25) (layer "F.Cu") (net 10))
 (segment (start 174.830825 70.98813) (end 171.277401 74.541554) (width 0.25) (layer "F.Cu") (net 8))
 (segment (start 174.830825 69.731045) (end 174.830825 70.98813) (width 0.25) (layer "F.Cu") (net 8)))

